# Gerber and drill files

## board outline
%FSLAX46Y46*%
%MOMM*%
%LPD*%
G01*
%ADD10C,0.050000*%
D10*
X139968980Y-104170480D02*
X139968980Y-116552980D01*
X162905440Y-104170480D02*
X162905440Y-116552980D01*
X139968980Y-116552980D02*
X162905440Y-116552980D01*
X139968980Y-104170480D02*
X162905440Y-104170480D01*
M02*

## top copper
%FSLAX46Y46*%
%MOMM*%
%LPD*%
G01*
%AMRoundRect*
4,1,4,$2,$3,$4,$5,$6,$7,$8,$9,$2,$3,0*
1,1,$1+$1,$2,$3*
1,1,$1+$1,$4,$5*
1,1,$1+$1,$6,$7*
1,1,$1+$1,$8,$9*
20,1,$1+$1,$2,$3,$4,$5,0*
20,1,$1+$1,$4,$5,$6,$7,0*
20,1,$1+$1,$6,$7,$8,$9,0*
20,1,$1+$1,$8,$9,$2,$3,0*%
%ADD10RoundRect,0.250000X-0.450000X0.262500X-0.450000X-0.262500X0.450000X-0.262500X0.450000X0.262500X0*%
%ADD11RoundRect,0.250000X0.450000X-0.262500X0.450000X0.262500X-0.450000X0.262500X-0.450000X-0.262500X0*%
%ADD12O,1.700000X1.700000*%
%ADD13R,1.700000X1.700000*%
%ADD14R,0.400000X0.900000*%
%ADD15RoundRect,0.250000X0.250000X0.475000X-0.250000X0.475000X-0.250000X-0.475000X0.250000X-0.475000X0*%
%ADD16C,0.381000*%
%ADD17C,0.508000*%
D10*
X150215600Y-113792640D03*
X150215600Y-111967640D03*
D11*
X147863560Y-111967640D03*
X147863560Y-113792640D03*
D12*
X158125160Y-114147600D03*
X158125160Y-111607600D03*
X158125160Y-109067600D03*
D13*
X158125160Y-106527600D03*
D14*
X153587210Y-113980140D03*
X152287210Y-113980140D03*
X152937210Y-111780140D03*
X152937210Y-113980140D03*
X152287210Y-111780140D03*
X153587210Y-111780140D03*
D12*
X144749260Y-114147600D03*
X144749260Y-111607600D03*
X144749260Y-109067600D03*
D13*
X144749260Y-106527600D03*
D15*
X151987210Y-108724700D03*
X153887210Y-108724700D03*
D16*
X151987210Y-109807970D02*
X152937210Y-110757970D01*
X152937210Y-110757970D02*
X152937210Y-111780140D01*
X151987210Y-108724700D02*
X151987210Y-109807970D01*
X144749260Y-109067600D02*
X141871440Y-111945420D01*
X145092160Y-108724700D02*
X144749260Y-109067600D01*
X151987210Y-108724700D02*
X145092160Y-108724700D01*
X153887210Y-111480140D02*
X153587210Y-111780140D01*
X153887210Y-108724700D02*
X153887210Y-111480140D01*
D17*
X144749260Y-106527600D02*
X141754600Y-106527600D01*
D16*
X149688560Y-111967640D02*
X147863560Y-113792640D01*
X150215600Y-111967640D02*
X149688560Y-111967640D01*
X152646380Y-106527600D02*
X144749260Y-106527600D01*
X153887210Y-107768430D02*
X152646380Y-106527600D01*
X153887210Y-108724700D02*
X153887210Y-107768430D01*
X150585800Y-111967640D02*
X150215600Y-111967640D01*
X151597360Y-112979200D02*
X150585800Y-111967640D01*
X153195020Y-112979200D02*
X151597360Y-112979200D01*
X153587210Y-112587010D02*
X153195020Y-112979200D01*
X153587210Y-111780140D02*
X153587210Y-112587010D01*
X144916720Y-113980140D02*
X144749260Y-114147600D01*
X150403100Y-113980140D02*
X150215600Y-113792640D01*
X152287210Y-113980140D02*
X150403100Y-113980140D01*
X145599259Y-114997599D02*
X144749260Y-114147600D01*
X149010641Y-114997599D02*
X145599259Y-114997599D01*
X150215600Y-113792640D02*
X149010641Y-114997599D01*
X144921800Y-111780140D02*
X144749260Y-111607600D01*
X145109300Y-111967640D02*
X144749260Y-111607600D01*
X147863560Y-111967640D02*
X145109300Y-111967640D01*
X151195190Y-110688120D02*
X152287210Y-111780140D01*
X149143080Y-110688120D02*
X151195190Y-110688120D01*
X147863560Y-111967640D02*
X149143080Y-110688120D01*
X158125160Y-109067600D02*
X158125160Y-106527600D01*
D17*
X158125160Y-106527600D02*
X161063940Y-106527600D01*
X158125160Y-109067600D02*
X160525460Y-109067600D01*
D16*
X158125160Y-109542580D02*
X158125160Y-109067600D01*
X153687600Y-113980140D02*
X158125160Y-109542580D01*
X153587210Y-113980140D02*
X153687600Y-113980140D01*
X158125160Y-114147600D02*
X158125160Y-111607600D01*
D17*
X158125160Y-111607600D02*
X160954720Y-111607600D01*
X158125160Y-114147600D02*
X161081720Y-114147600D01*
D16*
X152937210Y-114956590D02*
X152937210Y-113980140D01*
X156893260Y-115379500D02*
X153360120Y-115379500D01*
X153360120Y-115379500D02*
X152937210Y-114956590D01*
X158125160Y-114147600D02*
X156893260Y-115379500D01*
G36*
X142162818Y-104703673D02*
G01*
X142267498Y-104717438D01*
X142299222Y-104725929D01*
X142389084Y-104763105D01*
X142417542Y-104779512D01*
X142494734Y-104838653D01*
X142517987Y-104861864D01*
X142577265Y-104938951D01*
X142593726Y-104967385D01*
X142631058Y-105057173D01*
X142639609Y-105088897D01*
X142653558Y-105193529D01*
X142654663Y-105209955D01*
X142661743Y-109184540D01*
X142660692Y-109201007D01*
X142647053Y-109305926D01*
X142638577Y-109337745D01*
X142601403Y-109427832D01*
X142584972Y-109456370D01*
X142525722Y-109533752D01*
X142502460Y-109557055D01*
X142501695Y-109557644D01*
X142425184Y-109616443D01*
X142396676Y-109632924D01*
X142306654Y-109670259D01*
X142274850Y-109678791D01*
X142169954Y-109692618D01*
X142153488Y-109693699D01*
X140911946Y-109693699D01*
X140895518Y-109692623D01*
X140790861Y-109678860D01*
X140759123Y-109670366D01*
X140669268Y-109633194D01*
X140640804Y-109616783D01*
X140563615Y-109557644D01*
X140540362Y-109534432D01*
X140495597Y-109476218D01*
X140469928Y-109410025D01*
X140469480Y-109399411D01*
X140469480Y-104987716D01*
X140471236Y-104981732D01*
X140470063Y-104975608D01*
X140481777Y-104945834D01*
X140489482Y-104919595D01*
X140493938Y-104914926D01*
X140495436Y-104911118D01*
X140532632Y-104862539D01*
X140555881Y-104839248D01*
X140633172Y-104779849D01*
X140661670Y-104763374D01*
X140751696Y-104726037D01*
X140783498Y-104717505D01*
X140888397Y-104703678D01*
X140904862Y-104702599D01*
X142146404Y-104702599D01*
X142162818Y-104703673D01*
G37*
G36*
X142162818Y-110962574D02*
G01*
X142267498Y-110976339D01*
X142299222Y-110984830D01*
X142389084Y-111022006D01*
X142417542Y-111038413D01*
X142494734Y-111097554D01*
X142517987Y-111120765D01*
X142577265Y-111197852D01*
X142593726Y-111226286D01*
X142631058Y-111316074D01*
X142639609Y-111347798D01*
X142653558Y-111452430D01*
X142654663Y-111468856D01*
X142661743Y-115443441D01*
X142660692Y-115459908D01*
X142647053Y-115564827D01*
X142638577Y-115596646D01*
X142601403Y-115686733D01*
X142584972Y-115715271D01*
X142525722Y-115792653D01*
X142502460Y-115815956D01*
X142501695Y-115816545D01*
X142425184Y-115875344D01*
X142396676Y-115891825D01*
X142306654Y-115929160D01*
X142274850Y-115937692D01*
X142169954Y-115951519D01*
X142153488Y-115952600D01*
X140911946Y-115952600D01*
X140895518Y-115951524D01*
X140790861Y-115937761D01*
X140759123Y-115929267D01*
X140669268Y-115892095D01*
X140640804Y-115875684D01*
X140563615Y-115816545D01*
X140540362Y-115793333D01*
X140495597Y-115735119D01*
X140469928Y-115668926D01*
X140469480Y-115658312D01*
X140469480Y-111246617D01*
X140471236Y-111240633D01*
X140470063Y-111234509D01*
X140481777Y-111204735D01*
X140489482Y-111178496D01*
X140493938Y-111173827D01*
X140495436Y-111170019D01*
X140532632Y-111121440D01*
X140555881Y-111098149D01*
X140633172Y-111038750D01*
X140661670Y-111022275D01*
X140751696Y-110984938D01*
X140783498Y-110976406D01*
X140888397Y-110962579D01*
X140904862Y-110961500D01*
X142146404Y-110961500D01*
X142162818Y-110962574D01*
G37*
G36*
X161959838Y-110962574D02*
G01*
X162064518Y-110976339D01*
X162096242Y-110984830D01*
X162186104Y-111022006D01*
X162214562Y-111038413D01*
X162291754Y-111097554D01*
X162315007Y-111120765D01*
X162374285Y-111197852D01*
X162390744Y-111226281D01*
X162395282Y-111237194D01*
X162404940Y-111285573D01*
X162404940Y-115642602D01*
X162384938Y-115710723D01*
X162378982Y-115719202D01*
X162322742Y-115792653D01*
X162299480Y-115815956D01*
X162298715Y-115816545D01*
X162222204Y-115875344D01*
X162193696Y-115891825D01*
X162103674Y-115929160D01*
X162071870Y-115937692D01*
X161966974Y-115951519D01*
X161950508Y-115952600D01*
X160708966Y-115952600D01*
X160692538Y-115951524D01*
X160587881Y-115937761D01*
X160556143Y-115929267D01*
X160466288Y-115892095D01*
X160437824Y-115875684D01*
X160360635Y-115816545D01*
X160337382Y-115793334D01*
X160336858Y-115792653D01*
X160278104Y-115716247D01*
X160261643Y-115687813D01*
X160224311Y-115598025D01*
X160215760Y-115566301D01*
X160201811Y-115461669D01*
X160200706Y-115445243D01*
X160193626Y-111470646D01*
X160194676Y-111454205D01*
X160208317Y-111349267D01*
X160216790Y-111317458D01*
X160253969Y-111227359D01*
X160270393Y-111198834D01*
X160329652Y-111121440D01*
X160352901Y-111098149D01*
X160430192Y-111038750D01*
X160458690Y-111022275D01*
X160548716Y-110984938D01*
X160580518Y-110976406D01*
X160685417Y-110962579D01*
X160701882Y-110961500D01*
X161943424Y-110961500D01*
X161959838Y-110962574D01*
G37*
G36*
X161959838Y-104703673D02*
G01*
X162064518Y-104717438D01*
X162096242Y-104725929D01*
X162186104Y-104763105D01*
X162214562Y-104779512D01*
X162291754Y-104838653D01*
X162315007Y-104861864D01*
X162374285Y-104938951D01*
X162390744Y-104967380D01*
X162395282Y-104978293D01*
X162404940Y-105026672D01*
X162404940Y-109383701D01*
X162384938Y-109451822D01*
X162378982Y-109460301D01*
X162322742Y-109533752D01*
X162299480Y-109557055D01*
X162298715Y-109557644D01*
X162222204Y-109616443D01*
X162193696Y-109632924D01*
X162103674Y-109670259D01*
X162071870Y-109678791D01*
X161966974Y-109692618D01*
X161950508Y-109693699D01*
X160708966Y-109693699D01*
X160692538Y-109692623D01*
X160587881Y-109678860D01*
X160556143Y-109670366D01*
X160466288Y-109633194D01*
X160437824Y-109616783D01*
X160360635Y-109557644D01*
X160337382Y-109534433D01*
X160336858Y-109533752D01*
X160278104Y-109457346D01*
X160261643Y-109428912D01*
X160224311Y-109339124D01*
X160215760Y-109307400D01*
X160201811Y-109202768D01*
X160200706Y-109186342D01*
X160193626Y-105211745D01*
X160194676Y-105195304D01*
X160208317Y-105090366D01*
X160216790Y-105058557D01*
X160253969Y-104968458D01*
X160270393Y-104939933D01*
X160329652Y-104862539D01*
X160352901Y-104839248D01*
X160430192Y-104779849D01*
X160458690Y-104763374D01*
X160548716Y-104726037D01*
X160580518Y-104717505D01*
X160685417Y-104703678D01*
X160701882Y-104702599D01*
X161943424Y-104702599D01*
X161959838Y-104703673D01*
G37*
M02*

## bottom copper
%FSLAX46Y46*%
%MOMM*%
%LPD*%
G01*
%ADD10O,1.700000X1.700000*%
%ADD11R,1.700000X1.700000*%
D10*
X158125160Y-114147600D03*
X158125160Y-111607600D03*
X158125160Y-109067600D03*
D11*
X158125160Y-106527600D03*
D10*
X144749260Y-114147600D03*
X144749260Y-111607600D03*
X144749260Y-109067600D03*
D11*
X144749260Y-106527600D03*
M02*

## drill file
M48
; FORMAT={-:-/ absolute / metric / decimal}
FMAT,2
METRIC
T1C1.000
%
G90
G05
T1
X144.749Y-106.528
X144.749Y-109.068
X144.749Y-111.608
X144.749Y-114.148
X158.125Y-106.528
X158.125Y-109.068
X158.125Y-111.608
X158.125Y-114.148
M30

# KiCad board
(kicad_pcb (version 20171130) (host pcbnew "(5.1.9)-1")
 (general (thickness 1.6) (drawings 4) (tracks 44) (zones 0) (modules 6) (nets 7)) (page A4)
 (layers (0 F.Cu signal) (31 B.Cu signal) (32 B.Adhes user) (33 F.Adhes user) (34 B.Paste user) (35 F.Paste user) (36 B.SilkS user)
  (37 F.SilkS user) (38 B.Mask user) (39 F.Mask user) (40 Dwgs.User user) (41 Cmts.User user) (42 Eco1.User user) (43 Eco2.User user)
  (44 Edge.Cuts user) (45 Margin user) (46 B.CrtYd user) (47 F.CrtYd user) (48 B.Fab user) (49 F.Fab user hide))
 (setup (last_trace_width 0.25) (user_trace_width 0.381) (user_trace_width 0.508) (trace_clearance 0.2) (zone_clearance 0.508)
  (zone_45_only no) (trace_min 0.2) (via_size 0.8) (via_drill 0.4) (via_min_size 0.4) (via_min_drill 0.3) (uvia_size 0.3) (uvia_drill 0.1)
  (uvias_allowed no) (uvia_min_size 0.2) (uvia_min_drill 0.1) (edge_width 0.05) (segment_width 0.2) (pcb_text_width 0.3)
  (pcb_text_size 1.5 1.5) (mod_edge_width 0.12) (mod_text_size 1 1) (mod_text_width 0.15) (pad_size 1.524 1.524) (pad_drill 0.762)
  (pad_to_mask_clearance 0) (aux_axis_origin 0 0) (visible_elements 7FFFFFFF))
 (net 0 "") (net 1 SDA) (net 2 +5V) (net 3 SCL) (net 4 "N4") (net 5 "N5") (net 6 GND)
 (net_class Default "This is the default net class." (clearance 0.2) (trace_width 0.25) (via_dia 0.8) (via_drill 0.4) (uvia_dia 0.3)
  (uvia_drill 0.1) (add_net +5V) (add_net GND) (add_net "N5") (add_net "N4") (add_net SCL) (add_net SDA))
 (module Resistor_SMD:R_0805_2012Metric (layer F.Cu) (at 150.2156 112.88014 270)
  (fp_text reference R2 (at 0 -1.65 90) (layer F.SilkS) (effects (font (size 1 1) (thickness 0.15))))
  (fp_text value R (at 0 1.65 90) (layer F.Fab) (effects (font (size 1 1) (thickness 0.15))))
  (pad 2 smd roundrect (at 0.9125 0 270) (size 1.025 1.4) (layers F.Cu F.Paste F.Mask) (roundrect_rratio 0.243902) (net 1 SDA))
  (pad 1 smd roundrect (at -0.9125 0 270) (size 1.025 1.4) (layers F.Cu F.Paste F.Mask) (roundrect_rratio 0.243902) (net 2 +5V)))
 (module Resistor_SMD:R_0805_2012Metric (layer F.Cu) (at 147.86356 112.88014 90)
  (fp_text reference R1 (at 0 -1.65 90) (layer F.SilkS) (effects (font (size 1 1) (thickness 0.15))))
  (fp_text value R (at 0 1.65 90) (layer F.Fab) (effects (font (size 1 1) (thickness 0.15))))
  (pad 2 smd roundrect (at 0.9125 0 90) (size 1.025 1.4) (layers F.Cu F.Paste F.Mask) (roundrect_rratio 0.243902) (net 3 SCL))
  (pad 1 smd roundrect (at -0.9125 0 90) (size 1.025 1.4) (layers F.Cu F.Paste F.Mask) (roundrect_rratio 0.243902) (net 2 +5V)))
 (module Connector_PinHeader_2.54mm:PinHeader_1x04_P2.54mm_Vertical (layer F.Cu) (at 158.12516 106.5276)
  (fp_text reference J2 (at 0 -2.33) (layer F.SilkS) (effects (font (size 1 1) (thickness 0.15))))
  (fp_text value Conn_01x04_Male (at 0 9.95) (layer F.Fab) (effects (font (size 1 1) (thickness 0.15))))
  (pad 4 thru_hole oval (at 0 7.62) (size 1.7 1.7) (drill 1) (layers *.Cu *.Mask) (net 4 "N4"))
  (pad 3 thru_hole oval (at 0 5.08) (size 1.7 1.7) (drill 1) (layers *.Cu *.Mask) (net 4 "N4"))
  (pad 2 thru_hole oval (at 0 2.54) (size 1.7 1.7) (drill 1) (layers *.Cu *.Mask) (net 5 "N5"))
  (pad 1 thru_hole rect (at 0 0) (size 1.7 1.7) (drill 1) (layers *.Cu *.Mask) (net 5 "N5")))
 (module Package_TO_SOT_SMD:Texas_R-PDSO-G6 (layer F.Cu) (at 152.93721 112.88014 270)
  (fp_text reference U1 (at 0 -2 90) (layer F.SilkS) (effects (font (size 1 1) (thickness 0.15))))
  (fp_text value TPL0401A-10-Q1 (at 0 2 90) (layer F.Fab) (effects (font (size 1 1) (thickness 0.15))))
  (pad 6 smd rect (at 1.1 -0.65 270) (size 0.9 0.4) (layers F.Cu F.Paste F.Mask) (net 5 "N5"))
  (pad 4 smd rect (at 1.1 0.65 270) (size 0.9 0.4) (layers F.Cu F.Paste F.Mask) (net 1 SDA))
  (pad 2 smd rect (at -1.1 0 270) (size 0.9 0.4) (layers F.Cu F.Paste F.Mask) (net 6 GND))
  (pad 5 smd rect (at 1.1 0 270) (size 0.9 0.4) (layers F.Cu F.Paste F.Mask) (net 4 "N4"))
  (pad 3 smd rect (at -1.1 0.65 270) (size 0.9 0.4) (layers F.Cu F.Paste F.Mask) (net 3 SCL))
  (pad 1 smd rect (at -1.1 -0.65 270) (size 0.9 0.4) (layers F.Cu F.Paste F.Mask) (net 2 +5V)))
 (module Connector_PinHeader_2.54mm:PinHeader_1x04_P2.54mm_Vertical (layer F.Cu) (at 144.74926 106.5276)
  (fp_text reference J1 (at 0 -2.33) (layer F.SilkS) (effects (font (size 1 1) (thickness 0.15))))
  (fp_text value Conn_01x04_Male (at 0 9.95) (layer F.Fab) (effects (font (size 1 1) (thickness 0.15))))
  (pad 4 thru_hole oval (at 0 7.62) (size 1.7 1.7) (drill 1) (layers *.Cu *.Mask) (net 1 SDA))
  (pad 3 thru_hole oval (at 0 5.08) (size 1.7 1.7) (drill 1) (layers *.Cu *.Mask) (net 3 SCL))
  (pad 2 thru_hole oval (at 0 2.54) (size 1.7 1.7) (drill 1) (layers *.Cu *.Mask) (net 6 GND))
  (pad 1 thru_hole rect (at 0 0) (size 1.7 1.7) (drill 1) (layers *.Cu *.Mask) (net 2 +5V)))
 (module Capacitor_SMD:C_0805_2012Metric (layer F.Cu) (at 152.93721 108.7247 180)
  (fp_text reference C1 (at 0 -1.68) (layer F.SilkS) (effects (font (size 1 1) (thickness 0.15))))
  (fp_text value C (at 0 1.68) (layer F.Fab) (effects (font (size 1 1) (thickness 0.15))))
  (pad 2 smd roundrect (at 0.95 0 180) (size 1 1.45) (layers F.Cu F.Paste F.Mask) (roundrect_rratio 0.25) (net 6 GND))
  (pad 1 smd roundrect (at -0.95 0 180) (size 1 1.45) (layers F.Cu F.Paste F.Mask) (roundrect_rratio 0.25) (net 2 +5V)))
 (gr_line (start 139.96898 104.17048) (end 139.96898 116.55298) (layer Edge.Cuts) (width 0.05))
 (gr_line (start 162.90544 104.17048) (end 162.90544 116.55298) (layer Edge.Cuts) (width 0.05))
 (gr_line (start 139.96898 116.55298) (end 162.90544 116.55298) (layer Edge.Cuts) (width 0.05))
 (gr_line (start 139.96898 104.17048) (end 162.90544 104.17048) (layer Edge.Cuts) (width 0.05))
 (segment (start 151.98721 109.80797) (end 152.93721 110.75797) (width 0.381) (layer F.Cu) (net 6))
 (segment (start 152.93721 110.75797) (end 152.93721 111.78014) (width 0.381) (layer F.Cu) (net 6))
 (segment (start 151.98721 108.7247) (end 151.98721 109.80797) (width 0.381) (layer F.Cu) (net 6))
 (segment (start 144.74926 109.0676) (end 141.87144 111.94542) (width 0.381) (layer F.Cu) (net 6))
 (segment (start 145.09216 108.7247) (end 144.74926 109.0676) (width 0.381) (layer F.Cu) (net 6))
 (segment (start 151.98721 108.7247) (end 145.09216 108.7247) (width 0.381) (layer F.Cu) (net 6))
 (segment (start 153.88721 111.48014) (end 153.58721 111.78014) (width 0.381) (layer F.Cu) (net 2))
 (segment (start 153.88721 108.7247) (end 153.88721 111.48014) (width 0.381) (layer F.Cu) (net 2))
 (segment (start 144.74926 106.5276) (end 141.7546 106.5276) (width 0.508) (layer F.Cu) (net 2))
 (segment (start 149.68856 111.96764) (end 147.86356 113.79264) (width 0.381) (layer F.Cu) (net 2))
 (segment (start 150.2156 111.96764) (end 149.68856 111.96764) (width 0.381) (layer F.Cu) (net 2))
 (segment (start 152.64638 106.5276) (end 144.74926 106.5276) (width 0.381) (layer F.Cu) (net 2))
 (segment (start 153.88721 107.76843) (end 152.64638 106.5276) (width 0.381) (layer F.Cu) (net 2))
 (segment (start 153.88721 108.7247) (end 153.88721 107.76843) (width 0.381) (layer F.Cu) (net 2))
 (segment (start 150.5858 111.96764) (end 150.2156 111.96764) (width 0.381) (layer F.Cu) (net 2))
 (segment (start 151.59736 112.9792) (end 150.5858 111.96764) (width 0.381) (layer F.Cu) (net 2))
 (segment (start 153.19502 112.9792) (end 151.59736 112.9792) (width 0.381) (layer F.Cu) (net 2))
 (segment (start 153.58721 112.58701) (end 153.19502 112.9792) (width 0.381) (layer F.Cu) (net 2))
 (segment (start 153.58721 111.78014) (end 153.58721 112.58701) (width 0.381) (layer F.Cu) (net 2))
 (segment (start 144.91672 113.98014) (end 144.74926 114.1476) (width 0.381) (layer F.Cu) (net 1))
 (segment (start 150.4031 113.98014) (end 150.2156 113.79264) (width 0.381) (layer F.Cu) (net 1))
 (segment (start 152.28721 113.98014) (end 150.4031 113.98014) (width 0.381) (layer F.Cu) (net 1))
 (segment (start 145.599259 114.997599) (end 144.74926 114.1476) (width 0.381) (layer F.Cu) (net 1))
 (segment (start 149.010641 114.997599) (end 145.599259 114.997599) (width 0.381) (layer F.Cu) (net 1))
 (segment (start 150.2156 113.79264) (end 149.010641 114.997599) (width 0.381) (layer F.Cu) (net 1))
 (segment (start 144.9218 111.78014) (end 144.74926 111.6076) (width 0.381) (layer F.Cu) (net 3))
 (segment (start 145.1093 111.96764) (end 144.74926 111.6076) (width 0.381) (layer F.Cu) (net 3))
 (segment (start 147.86356 111.96764) (end 145.1093 111.96764) (width 0.381) (layer F.Cu) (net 3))
 (segment (start 151.19519 110.68812) (end 152.28721 111.78014) (width 0.381) (layer F.Cu) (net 3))
 (segment (start 149.14308 110.68812) (end 151.19519 110.68812) (width 0.381) (layer F.Cu) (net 3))
 (segment (start 147.86356 111.96764) (end 149.14308 110.68812) (width 0.381) (layer F.Cu) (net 3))
 (segment (start 158.12516 109.0676) (end 158.12516 106.5276) (width 0.381) (layer F.Cu) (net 5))
 (segment (start 158.12516 106.5276) (end 161.06394 106.5276) (width 0.508) (layer F.Cu) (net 5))
 (segment (start 158.12516 109.0676) (end 160.52546 109.0676) (width 0.508) (layer F.Cu) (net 5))
 (segment (start 158.12516 109.54258) (end 158.12516 109.0676) (width 0.381) (layer F.Cu) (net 5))
 (segment (start 153.6876 113.98014) (end 158.12516 109.54258) (width 0.381) (layer F.Cu) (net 5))
 (segment (start 153.58721 113.98014) (end 153.6876 113.98014) (width 0.381) (layer F.Cu) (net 5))
 (segment (start 158.12516 114.1476) (end 158.12516 111.6076) (width 0.381) (layer F.Cu) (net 4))
 (segment (start 158.12516 111.6076) (end 160.95472 111.6076) (width 0.508) (layer F.Cu) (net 4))
 (segment (start 158.12516 114.1476) (end 161.08172 114.1476) (width 0.508) (layer F.Cu) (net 4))
 (segment (start 152.93721 114.95659) (end 152.93721 113.98014) (width 0.381) (layer F.Cu) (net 4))
 (segment (start 156.89326 115.3795) (end 153.36012 115.3795) (width 0.381) (layer F.Cu) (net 4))
 (segment (start 153.36012 115.3795) (end 152.93721 114.95659) (width 0.381) (layer F.Cu) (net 4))
 (segment (start 158.12516 114.1476) (end 156.89326 115.3795) (width 0.381) (layer F.Cu) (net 4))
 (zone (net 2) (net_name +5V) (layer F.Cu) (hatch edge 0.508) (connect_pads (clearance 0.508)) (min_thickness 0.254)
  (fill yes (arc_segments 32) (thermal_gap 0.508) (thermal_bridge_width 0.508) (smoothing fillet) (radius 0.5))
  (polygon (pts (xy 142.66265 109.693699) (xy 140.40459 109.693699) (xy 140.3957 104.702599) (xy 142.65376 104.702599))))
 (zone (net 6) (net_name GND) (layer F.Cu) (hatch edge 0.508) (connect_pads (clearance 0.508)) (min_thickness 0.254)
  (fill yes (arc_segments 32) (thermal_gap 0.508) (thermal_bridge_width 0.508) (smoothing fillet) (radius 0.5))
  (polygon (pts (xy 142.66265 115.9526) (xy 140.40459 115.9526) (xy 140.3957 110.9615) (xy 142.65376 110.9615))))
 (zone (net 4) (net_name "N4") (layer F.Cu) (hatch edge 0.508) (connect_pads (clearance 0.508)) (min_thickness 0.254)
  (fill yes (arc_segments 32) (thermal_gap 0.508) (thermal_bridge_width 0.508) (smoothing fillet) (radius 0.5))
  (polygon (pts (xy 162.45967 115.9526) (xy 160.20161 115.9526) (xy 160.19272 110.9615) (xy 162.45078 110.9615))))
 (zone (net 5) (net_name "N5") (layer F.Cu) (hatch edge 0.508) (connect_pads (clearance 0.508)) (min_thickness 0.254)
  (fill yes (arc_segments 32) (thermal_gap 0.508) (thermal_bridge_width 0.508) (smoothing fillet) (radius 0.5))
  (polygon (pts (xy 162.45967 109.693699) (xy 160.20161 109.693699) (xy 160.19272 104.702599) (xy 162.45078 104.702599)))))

